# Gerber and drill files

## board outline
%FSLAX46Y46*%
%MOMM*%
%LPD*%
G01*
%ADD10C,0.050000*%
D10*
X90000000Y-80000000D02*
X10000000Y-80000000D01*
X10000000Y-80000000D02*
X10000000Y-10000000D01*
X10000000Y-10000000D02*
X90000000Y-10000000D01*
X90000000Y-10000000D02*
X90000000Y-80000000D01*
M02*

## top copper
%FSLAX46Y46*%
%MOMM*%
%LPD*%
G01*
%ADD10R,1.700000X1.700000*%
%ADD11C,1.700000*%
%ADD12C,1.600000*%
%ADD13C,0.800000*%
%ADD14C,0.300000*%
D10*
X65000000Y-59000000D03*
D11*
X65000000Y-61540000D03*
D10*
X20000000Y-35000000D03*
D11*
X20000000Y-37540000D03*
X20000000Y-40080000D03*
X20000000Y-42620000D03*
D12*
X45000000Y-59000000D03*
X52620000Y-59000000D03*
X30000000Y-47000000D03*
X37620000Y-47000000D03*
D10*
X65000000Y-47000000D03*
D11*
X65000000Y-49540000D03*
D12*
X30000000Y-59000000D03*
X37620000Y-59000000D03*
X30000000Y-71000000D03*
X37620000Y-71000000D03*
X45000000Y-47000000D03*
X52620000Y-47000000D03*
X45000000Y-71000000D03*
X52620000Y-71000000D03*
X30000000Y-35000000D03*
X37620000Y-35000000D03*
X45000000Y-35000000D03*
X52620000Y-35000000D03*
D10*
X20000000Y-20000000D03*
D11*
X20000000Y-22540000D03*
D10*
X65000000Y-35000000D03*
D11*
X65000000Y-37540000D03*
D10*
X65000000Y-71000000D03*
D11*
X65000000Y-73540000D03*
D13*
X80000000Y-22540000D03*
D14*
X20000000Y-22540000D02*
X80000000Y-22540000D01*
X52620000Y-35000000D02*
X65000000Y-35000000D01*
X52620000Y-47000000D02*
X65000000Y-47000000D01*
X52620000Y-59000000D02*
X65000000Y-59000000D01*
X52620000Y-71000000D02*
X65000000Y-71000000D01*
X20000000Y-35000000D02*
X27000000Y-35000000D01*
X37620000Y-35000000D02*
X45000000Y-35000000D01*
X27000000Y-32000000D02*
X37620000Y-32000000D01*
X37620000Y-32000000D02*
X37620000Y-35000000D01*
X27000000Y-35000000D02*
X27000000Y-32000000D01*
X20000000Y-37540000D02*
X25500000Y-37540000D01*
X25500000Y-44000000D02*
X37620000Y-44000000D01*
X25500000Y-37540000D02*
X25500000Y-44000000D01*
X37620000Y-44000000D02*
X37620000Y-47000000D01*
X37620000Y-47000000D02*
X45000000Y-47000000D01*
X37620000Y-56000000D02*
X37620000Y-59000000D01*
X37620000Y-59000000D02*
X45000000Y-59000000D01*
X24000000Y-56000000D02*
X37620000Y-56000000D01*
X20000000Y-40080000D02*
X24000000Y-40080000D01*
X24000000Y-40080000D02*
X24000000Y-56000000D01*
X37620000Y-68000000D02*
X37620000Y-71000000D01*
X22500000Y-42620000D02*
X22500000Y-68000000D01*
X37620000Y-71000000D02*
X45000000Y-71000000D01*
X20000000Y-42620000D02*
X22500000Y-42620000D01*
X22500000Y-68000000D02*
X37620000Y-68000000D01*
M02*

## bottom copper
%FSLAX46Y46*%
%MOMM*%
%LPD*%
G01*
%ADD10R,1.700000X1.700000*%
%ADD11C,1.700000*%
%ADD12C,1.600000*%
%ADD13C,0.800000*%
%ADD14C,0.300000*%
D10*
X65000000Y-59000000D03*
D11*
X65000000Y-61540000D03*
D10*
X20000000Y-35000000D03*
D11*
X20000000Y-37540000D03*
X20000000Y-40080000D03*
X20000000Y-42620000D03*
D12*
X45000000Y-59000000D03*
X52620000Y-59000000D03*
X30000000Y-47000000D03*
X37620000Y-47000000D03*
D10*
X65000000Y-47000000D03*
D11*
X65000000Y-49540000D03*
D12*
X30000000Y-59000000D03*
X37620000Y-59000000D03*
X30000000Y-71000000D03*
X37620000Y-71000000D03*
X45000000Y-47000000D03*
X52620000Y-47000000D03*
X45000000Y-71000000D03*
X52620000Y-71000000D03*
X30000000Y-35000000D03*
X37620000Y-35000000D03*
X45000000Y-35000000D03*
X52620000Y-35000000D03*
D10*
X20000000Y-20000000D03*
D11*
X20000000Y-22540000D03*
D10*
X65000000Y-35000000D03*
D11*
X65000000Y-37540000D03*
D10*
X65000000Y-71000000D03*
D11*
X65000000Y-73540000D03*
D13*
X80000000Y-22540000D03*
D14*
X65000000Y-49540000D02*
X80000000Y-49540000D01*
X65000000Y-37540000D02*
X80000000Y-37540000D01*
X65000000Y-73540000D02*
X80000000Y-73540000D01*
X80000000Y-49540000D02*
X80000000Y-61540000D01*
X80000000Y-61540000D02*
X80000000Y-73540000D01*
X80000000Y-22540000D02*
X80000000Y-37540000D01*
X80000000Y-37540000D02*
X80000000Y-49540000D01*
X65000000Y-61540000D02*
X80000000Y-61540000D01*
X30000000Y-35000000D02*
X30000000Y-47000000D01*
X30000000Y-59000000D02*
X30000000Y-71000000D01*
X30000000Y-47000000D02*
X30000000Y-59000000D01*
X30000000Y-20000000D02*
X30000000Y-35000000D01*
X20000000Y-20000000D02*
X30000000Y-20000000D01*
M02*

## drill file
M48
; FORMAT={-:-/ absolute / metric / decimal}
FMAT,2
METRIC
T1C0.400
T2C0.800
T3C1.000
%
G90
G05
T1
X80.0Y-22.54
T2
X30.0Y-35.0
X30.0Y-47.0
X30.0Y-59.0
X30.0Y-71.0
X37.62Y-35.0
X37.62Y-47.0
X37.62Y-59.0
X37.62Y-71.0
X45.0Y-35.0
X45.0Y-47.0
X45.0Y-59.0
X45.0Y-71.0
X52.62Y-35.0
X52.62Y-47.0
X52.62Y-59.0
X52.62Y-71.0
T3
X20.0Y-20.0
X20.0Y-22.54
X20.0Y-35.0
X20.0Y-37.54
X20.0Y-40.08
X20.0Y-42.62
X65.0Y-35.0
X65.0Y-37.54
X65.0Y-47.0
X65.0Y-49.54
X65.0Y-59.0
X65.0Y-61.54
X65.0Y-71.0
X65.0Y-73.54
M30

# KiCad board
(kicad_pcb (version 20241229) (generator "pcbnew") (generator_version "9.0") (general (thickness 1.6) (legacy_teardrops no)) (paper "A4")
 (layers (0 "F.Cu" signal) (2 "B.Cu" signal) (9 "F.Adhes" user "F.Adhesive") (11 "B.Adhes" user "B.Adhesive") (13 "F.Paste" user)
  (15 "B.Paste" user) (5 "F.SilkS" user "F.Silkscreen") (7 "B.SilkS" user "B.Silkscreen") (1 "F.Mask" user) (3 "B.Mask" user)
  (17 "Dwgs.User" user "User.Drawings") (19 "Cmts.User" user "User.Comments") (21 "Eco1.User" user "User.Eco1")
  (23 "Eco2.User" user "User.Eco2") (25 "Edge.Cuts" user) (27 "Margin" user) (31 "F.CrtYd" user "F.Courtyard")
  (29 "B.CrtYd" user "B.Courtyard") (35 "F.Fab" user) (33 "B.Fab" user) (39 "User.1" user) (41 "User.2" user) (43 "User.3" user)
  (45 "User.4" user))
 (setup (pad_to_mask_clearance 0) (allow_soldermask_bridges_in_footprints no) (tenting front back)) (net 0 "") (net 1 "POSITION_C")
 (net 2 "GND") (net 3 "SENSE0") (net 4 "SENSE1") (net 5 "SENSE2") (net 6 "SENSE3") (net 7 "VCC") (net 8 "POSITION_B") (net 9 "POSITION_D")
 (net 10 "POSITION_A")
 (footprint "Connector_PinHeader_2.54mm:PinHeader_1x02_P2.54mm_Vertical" (layer "F.Cu") (at 65 59)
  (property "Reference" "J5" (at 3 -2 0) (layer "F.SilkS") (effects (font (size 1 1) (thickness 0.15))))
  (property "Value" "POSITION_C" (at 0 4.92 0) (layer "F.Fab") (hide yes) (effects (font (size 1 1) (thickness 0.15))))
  (pad "1" thru_hole rect (at 0 0) (size 1.7 1.7) (drill 1) (layers "*.Cu" "*.Mask") (remove_unused_layers no) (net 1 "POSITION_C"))
  (pad "2" thru_hole circle (at 0 2.54) (size 1.7 1.7) (drill 1) (layers "*.Cu" "*.Mask") (remove_unused_layers no) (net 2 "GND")))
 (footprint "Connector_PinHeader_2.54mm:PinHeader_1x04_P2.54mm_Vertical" (layer "F.Cu") (at 20 35)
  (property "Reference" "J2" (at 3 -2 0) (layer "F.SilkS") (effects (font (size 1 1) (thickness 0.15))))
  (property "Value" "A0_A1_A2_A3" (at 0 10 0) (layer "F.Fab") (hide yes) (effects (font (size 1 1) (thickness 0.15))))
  (pad "1" thru_hole rect (at 0 0) (size 1.7 1.7) (drill 1) (layers "*.Cu" "*.Mask") (remove_unused_layers no) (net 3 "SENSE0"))
  (pad "2" thru_hole circle (at 0 2.54) (size 1.7 1.7) (drill 1) (layers "*.Cu" "*.Mask") (remove_unused_layers no) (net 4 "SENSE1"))
  (pad "3" thru_hole circle (at 0 5.08) (size 1.7 1.7) (drill 1) (layers "*.Cu" "*.Mask") (remove_unused_layers no) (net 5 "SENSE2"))
  (pad "4" thru_hole circle (at 0 7.62) (size 1.7 1.7) (drill 1) (layers "*.Cu" "*.Mask") (remove_unused_layers no) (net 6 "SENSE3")))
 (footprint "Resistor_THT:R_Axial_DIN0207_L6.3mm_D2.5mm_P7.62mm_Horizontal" (layer "F.Cu") (at 45 59)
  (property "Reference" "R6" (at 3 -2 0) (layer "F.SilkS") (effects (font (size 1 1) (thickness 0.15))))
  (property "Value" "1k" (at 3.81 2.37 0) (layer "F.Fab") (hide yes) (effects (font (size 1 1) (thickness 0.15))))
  (pad "1" thru_hole circle (at 0 0) (size 1.6 1.6) (drill 0.8) (layers "*.Cu" "*.Mask") (remove_unused_layers no) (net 5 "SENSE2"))
  (pad "2" thru_hole circle (at 7.62 0) (size 1.6 1.6) (drill 0.8) (layers "*.Cu" "*.Mask") (remove_unused_layers no) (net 1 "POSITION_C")))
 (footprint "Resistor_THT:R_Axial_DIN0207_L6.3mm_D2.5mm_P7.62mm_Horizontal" (layer "F.Cu") (at 30 47)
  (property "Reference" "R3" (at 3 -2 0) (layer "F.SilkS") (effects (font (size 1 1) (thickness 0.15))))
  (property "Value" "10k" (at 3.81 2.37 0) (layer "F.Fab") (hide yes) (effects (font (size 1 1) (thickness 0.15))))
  (pad "1" thru_hole circle (at 0 0) (size 1.6 1.6) (drill 0.8) (layers "*.Cu" "*.Mask") (remove_unused_layers no) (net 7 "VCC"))
  (pad "2" thru_hole circle (at 7.62 0) (size 1.6 1.6) (drill 0.8) (layers "*.Cu" "*.Mask") (remove_unused_layers no) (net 4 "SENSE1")))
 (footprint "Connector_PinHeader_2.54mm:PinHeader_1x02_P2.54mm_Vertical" (layer "F.Cu") (at 65 47)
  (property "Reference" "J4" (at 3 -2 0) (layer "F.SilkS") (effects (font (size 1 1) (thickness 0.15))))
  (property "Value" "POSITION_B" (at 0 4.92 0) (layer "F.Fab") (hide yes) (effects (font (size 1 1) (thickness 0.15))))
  (pad "1" thru_hole rect (at 0 0) (size 1.7 1.7) (drill 1) (layers "*.Cu" "*.Mask") (remove_unused_layers no) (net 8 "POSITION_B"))
  (pad "2" thru_hole circle (at 0 2.54) (size 1.7 1.7) (drill 1) (layers "*.Cu" "*.Mask") (remove_unused_layers no) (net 2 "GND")))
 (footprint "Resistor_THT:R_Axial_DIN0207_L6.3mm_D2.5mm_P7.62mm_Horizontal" (layer "F.Cu") (at 30 59)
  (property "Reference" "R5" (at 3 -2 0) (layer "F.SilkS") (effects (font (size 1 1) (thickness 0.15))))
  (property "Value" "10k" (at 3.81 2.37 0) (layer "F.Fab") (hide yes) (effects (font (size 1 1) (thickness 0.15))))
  (pad "1" thru_hole circle (at 0 0) (size 1.6 1.6) (drill 0.8) (layers "*.Cu" "*.Mask") (remove_unused_layers no) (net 7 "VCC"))
  (pad "2" thru_hole circle (at 7.62 0) (size 1.6 1.6) (drill 0.8) (layers "*.Cu" "*.Mask") (remove_unused_layers no) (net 5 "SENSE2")))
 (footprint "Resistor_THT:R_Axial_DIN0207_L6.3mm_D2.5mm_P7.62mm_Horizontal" (layer "F.Cu") (at 30 71)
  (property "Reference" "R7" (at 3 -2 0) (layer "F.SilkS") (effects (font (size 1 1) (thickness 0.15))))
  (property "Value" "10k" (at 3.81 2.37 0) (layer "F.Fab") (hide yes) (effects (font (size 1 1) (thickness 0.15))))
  (pad "1" thru_hole circle (at 0 0) (size 1.6 1.6) (drill 0.8) (layers "*.Cu" "*.Mask") (remove_unused_layers no) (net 7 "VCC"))
  (pad "2" thru_hole circle (at 7.62 0) (size 1.6 1.6) (drill 0.8) (layers "*.Cu" "*.Mask") (remove_unused_layers no) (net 6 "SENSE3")))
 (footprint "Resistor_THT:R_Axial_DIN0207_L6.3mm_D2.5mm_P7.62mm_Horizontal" (layer "F.Cu") (at 45 47)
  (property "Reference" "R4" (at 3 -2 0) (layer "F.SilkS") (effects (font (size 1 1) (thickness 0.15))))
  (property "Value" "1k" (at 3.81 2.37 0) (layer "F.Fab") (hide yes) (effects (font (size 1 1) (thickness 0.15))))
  (pad "1" thru_hole circle (at 0 0) (size 1.6 1.6) (drill 0.8) (layers "*.Cu" "*.Mask") (remove_unused_layers no) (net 4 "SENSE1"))
  (pad "2" thru_hole circle (at 7.62 0) (size 1.6 1.6) (drill 0.8) (layers "*.Cu" "*.Mask") (remove_unused_layers no) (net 8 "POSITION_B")))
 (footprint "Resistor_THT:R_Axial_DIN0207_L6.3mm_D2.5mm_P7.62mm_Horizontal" (layer "F.Cu") (at 45 71)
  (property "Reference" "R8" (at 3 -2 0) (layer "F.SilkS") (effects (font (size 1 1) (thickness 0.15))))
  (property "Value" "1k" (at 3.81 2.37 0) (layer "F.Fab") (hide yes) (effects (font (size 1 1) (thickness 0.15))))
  (pad "1" thru_hole circle (at 0 0) (size 1.6 1.6) (drill 0.8) (layers "*.Cu" "*.Mask") (remove_unused_layers no) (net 6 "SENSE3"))
  (pad "2" thru_hole circle (at 7.62 0) (size 1.6 1.6) (drill 0.8) (layers "*.Cu" "*.Mask") (remove_unused_layers no) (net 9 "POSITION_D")))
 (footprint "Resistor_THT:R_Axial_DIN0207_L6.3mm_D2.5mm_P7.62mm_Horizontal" (layer "F.Cu") (at 30 35)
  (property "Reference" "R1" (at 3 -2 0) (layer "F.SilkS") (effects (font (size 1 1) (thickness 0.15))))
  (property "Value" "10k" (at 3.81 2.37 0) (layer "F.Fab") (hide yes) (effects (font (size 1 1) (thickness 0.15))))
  (pad "1" thru_hole circle (at 0 0) (size 1.6 1.6) (drill 0.8) (layers "*.Cu" "*.Mask") (remove_unused_layers no) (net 7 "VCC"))
  (pad "2" thru_hole circle (at 7.62 0) (size 1.6 1.6) (drill 0.8) (layers "*.Cu" "*.Mask") (remove_unused_layers no) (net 3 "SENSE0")))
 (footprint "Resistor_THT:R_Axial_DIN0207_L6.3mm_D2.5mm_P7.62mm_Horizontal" (layer "F.Cu") (at 45 35)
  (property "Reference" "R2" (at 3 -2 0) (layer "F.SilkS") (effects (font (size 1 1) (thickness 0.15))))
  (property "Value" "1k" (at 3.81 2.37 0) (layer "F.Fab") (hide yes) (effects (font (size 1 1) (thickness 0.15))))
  (pad "1" thru_hole circle (at 0 0) (size 1.6 1.6) (drill 0.8) (layers "*.Cu" "*.Mask") (remove_unused_layers no) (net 3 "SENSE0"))
  (pad "2" thru_hole circle (at 7.62 0) (size 1.6 1.6) (drill 0.8) (layers "*.Cu" "*.Mask") (remove_unused_layers no) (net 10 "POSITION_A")))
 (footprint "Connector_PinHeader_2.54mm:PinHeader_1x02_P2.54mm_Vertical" (layer "F.Cu") (at 20 20)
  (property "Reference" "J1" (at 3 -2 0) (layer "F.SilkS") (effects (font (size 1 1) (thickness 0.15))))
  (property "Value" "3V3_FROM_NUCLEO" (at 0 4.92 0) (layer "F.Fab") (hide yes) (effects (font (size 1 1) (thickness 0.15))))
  (pad "1" thru_hole rect (at 0 0) (size 1.7 1.7) (drill 1) (layers "*.Cu" "*.Mask") (remove_unused_layers no) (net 7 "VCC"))
  (pad "2" thru_hole circle (at 0 2.54) (size 1.7 1.7) (drill 1) (layers "*.Cu" "*.Mask") (remove_unused_layers no) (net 2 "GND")))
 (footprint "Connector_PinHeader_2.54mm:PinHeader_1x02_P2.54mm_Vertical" (layer "F.Cu") (at 65 35)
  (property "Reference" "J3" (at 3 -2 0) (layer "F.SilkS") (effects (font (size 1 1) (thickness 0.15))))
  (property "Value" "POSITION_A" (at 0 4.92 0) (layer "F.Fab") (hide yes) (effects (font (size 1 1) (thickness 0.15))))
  (pad "1" thru_hole rect (at 0 0) (size 1.7 1.7) (drill 1) (layers "*.Cu" "*.Mask") (remove_unused_layers no) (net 10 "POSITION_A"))
  (pad "2" thru_hole circle (at 0 2.54) (size 1.7 1.7) (drill 1) (layers "*.Cu" "*.Mask") (remove_unused_layers no) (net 2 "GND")))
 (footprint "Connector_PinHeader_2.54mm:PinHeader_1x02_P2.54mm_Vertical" (layer "F.Cu") (at 65 71)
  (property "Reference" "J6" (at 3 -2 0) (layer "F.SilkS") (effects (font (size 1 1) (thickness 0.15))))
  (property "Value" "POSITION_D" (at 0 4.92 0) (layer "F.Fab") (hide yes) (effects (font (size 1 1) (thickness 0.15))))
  (pad "1" thru_hole rect (at 0 0) (size 1.7 1.7) (drill 1) (layers "*.Cu" "*.Mask") (remove_unused_layers no) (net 9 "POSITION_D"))
  (pad "2" thru_hole circle (at 0 2.54) (size 1.7 1.7) (drill 1) (layers "*.Cu" "*.Mask") (remove_unused_layers no) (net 2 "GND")))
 (gr_line (start 90 80) (end 10 80) (stroke (width 0.05) (type default)) (layer "Edge.Cuts"))
 (gr_line (start 10 80) (end 10 10) (stroke (width 0.05) (type default)) (layer "Edge.Cuts"))
 (gr_line (start 10 10) (end 90 10) (stroke (width 0.05) (type default)) (layer "Edge.Cuts"))
 (gr_line (start 90 10) (end 90 80) (stroke (width 0.05) (type default)) (layer "Edge.Cuts"))
 (segment (start 20 22.54) (end 80 22.54) (width 0.3) (layer "F.Cu") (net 2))
 (via (at 80 22.54) (size 0.8) (drill 0.4) (layers "F.Cu" "B.Cu") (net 2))
 (segment (start 65 49.54) (end 80 49.54) (width 0.3) (layer "B.Cu") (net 2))
 (segment (start 65 37.54) (end 80 37.54) (width 0.3) (layer "B.Cu") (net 2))
 (segment (start 65 73.54) (end 80 73.54) (width 0.3) (layer "B.Cu") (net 2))
 (segment (start 80 49.54) (end 80 61.54) (width 0.3) (layer "B.Cu") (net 2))
 (segment (start 80 61.54) (end 80 73.54) (width 0.3) (layer "B.Cu") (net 2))
 (segment (start 80 22.54) (end 80 37.54) (width 0.3) (layer "B.Cu") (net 2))
 (segment (start 80 37.54) (end 80 49.54) (width 0.3) (layer "B.Cu") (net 2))
 (segment (start 65 61.54) (end 80 61.54) (width 0.3) (layer "B.Cu") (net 2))
 (segment (start 52.62 35) (end 65 35) (width 0.3) (layer "F.Cu") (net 10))
 (segment (start 52.62 47) (end 65 47) (width 0.3) (layer "F.Cu") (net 8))
 (segment (start 52.62 59) (end 65 59) (width 0.3) (layer "F.Cu") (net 1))
 (segment (start 52.62 71) (end 65 71) (width 0.3) (layer "F.Cu") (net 9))
 (segment (start 20 35) (end 27 35) (width 0.3) (layer "F.Cu") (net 3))
 (segment (start 37.62 35) (end 45 35) (width 0.3) (layer "F.Cu") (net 3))
 (segment (start 27 32) (end 37.62 32) (width 0.3) (layer "F.Cu") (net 3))
 (segment (start 37.62 32) (end 37.62 35) (width 0.3) (layer "F.Cu") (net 3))
 (segment (start 27 35) (end 27 32) (width 0.3) (layer "F.Cu") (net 3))
 (segment (start 20 37.54) (end 25.5 37.54) (width 0.3) (layer "F.Cu") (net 4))
 (segment (start 25.5 44) (end 37.62 44) (width 0.3) (layer "F.Cu") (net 4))
 (segment (start 25.5 37.54) (end 25.5 44) (width 0.3) (layer "F.Cu") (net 4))
 (segment (start 37.62 44) (end 37.62 47) (width 0.3) (layer "F.Cu") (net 4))
 (segment (start 37.62 47) (end 45 47) (width 0.3) (layer "F.Cu") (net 4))
 (segment (start 37.62 56) (end 37.62 59) (width 0.3) (layer "F.Cu") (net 5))
 (segment (start 37.62 59) (end 45 59) (width 0.3) (layer "F.Cu") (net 5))
 (segment (start 24 56) (end 37.62 56) (width 0.3) (layer "F.Cu") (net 5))
 (segment (start 20 40.08) (end 24 40.08) (width 0.3) (layer "F.Cu") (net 5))
 (segment (start 24 40.08) (end 24 56) (width 0.3) (layer "F.Cu") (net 5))
 (segment (start 37.62 68) (end 37.62 71) (width 0.3) (layer "F.Cu") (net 6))
 (segment (start 22.5 42.62) (end 22.5 68) (width 0.3) (layer "F.Cu") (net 6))
 (segment (start 37.62 71) (end 45 71) (width 0.3) (layer "F.Cu") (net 6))
 (segment (start 20 42.62) (end 22.5 42.62) (width 0.3) (layer "F.Cu") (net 6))
 (segment (start 22.5 68) (end 37.62 68) (width 0.3) (layer "F.Cu") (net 6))
 (segment (start 30 35) (end 30 47) (width 0.3) (layer "B.Cu") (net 7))
 (segment (start 30 59) (end 30 71) (width 0.3) (layer "B.Cu") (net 7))
 (segment (start 30 47) (end 30 59) (width 0.3) (layer "B.Cu") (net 7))
 (segment (start 30 20) (end 30 35) (width 0.3) (layer "B.Cu") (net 7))
 (segment (start 20 20) (end 30 20) (width 0.3) (layer "B.Cu") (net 7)))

